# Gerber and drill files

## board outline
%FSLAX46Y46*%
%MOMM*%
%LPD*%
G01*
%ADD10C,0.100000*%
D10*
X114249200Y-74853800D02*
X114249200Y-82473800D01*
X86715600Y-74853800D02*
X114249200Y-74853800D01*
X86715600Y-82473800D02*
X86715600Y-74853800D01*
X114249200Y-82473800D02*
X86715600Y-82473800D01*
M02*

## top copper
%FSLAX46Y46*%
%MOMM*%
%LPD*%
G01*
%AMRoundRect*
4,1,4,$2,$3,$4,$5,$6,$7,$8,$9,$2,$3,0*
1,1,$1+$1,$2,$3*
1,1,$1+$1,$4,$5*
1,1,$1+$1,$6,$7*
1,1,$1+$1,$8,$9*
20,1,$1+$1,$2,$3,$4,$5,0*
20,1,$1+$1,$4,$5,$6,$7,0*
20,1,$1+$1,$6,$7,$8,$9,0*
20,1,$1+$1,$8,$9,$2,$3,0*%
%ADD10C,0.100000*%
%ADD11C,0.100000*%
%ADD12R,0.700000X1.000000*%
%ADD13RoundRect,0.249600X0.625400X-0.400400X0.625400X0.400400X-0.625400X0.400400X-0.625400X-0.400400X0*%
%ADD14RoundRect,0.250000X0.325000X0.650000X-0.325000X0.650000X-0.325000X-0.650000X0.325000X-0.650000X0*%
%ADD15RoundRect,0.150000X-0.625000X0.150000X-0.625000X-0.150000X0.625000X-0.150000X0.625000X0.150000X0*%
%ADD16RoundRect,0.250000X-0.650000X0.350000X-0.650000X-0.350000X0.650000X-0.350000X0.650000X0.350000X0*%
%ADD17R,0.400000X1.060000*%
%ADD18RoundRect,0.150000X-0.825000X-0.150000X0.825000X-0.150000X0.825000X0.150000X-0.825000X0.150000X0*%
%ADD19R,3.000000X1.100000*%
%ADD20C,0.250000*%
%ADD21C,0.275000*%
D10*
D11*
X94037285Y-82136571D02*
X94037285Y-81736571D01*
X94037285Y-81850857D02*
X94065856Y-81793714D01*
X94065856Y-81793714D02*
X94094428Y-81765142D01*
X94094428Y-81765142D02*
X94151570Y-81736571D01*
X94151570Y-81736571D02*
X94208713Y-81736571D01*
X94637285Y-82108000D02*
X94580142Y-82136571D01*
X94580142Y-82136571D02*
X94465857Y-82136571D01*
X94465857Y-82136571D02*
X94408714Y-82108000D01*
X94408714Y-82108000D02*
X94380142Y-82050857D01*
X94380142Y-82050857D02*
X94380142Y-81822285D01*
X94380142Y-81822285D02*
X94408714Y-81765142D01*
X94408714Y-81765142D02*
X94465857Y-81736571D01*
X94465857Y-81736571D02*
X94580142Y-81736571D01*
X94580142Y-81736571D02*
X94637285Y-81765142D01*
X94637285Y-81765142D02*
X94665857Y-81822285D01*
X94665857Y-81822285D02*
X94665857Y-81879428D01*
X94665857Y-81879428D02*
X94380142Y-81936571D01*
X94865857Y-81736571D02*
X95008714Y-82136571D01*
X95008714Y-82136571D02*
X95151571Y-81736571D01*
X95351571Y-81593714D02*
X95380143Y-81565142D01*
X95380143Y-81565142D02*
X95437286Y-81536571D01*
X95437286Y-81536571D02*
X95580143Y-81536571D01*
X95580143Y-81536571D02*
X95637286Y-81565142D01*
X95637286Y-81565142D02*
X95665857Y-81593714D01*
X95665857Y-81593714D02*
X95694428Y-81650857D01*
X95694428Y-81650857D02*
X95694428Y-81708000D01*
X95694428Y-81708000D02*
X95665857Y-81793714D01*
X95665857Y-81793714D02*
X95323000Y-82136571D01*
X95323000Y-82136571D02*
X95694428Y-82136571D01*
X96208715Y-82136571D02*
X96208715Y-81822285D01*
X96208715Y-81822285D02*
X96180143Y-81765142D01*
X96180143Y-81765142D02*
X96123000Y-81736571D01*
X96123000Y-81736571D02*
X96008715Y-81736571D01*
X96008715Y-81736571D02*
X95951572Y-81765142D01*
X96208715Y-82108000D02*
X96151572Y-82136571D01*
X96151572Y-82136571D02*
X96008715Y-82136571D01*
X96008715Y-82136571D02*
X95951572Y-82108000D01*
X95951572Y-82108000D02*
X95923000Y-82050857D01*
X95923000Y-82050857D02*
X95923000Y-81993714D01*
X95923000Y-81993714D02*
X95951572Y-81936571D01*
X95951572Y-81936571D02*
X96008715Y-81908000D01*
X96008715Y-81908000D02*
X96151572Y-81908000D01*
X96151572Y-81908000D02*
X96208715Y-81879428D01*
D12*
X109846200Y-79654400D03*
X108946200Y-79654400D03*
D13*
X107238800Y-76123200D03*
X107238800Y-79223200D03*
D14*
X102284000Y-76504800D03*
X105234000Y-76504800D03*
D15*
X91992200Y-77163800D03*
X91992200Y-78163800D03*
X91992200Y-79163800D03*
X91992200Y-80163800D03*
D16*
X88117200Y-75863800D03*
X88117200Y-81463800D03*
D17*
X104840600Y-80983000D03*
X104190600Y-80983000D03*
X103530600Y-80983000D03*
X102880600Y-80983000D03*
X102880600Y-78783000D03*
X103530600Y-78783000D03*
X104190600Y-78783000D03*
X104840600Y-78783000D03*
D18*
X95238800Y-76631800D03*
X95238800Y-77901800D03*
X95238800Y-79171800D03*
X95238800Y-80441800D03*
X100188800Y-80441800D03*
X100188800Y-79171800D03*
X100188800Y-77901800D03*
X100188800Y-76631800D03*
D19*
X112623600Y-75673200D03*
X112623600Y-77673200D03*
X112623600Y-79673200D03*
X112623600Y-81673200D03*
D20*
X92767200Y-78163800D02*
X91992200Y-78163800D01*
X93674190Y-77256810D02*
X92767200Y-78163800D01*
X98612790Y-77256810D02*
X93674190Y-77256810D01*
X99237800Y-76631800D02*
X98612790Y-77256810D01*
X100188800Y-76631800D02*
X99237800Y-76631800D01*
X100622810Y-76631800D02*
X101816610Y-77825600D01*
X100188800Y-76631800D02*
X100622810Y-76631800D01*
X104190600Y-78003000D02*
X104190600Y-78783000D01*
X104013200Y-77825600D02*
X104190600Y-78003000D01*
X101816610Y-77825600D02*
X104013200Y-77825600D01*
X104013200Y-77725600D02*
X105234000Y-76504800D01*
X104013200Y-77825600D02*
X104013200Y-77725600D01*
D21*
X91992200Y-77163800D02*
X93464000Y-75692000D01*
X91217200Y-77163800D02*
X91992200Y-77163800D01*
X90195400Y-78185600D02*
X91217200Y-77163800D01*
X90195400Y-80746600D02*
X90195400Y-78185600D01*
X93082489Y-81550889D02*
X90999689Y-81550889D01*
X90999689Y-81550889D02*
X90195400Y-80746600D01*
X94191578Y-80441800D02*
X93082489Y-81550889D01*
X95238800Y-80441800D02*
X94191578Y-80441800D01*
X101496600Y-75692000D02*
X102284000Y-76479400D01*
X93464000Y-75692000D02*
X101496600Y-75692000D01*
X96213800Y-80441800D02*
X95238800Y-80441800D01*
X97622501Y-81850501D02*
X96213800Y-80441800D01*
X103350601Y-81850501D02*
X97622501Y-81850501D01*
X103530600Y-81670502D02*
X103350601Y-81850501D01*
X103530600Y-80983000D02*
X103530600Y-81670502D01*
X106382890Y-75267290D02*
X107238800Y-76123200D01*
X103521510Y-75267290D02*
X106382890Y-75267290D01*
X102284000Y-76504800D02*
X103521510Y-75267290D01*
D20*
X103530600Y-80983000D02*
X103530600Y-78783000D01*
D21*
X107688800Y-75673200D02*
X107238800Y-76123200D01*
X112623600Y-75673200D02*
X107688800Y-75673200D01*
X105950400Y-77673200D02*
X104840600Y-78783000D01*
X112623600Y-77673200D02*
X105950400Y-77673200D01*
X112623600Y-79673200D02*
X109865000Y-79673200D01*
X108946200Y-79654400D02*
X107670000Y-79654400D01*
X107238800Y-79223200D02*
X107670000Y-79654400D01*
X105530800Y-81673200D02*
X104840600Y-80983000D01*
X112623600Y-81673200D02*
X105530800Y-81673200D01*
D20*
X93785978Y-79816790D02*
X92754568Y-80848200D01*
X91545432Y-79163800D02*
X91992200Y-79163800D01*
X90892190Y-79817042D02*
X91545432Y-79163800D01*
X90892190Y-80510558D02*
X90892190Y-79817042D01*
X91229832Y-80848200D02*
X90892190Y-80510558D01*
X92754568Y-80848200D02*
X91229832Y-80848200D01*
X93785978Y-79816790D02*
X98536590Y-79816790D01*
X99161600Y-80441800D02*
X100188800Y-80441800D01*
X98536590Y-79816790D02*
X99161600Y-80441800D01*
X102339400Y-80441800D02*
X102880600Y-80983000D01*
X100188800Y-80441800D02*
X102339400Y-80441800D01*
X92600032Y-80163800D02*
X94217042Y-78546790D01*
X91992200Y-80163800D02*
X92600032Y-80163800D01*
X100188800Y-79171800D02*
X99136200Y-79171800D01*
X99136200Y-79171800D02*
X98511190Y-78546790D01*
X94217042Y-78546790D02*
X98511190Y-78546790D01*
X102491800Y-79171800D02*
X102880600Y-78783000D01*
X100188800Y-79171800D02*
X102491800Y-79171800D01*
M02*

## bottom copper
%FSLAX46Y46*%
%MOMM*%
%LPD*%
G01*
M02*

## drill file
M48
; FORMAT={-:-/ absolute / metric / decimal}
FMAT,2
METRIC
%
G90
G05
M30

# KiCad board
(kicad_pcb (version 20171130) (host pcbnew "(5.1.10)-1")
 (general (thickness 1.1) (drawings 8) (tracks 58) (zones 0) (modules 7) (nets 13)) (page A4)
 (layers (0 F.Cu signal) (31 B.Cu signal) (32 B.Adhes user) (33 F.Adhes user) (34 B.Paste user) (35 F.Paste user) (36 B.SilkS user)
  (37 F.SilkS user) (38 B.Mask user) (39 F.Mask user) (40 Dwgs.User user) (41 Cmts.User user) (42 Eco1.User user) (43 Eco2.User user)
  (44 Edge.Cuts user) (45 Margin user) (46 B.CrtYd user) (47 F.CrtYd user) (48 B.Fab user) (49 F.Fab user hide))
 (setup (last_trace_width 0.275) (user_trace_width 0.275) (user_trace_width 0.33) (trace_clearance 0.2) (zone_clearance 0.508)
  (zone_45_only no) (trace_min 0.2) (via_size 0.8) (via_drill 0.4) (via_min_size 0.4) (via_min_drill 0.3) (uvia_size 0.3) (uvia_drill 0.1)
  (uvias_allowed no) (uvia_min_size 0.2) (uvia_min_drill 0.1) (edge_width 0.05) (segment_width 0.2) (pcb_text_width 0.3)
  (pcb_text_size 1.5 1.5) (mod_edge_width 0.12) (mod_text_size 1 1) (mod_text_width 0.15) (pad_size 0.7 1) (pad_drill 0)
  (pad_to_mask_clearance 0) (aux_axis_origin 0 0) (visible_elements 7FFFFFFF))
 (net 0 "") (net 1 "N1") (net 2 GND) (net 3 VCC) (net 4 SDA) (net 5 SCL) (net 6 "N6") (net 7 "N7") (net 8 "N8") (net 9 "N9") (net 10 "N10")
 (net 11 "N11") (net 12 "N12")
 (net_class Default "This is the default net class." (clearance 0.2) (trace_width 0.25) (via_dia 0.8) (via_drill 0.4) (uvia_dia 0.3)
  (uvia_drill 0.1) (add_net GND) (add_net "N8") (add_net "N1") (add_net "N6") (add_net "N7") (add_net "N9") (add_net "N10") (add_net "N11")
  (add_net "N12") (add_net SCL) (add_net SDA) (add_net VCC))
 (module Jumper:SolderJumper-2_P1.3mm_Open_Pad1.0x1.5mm (layer F.Cu) (at 109.2962 79.6544)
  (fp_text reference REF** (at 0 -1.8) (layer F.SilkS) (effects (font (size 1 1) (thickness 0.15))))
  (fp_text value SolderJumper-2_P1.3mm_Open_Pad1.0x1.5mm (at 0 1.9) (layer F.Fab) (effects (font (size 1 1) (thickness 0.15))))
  (pad 2 smd rect (at 0.55 0) (size 0.7 1) (layers F.Cu F.Mask) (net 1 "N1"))
  (pad 1 smd rect (at -0.35 0) (size 0.7 1) (layers F.Cu F.Mask) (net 1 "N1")))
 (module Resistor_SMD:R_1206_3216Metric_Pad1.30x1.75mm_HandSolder (layer F.Cu) (at 107.2388 77.6732 90)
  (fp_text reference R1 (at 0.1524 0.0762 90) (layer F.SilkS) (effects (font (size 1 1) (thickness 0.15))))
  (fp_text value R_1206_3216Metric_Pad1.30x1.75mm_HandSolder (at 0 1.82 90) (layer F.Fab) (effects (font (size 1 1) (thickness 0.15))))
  (pad 2 smd roundrect (at 1.55 0 90) (size 1.3 1.75) (layers F.Cu F.Paste F.Mask) (roundrect_rratio 0.192) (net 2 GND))
  (pad 1 smd roundrect (at -1.55 0 90) (size 1.3 1.75) (layers F.Cu F.Paste F.Mask) (roundrect_rratio 0.192) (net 1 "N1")))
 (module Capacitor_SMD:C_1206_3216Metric (layer F.Cu) (at 103.759 76.5048 180)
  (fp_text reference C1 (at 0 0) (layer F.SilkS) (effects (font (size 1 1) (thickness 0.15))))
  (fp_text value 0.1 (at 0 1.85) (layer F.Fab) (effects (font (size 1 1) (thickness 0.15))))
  (pad 2 smd roundrect (at 1.475 0 180) (size 1.15 1.8) (layers F.Cu F.Paste F.Mask) (roundrect_rratio 0.217391) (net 2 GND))
  (pad 1 smd roundrect (at -1.475 0 180) (size 1.15 1.8) (layers F.Cu F.Paste F.Mask) (roundrect_rratio 0.217391) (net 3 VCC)))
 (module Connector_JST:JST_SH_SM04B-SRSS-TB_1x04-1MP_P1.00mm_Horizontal (layer F.Cu) (at 89.9922 78.6638 270)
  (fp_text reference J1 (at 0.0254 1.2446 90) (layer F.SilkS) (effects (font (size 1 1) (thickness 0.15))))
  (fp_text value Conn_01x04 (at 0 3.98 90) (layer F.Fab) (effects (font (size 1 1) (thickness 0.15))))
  (pad 1 smd roundrect (at -1.5 -2 270) (size 0.6 1.55) (layers F.Cu F.Paste F.Mask) (roundrect_rratio 0.25) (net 2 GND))
  (pad 2 smd roundrect (at -0.5 -2 270) (size 0.6 1.55) (layers F.Cu F.Paste F.Mask) (roundrect_rratio 0.25) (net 3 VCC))
  (pad 3 smd roundrect (at 0.5 -2 270) (size 0.6 1.55) (layers F.Cu F.Paste F.Mask) (roundrect_rratio 0.25) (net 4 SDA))
  (pad 4 smd roundrect (at 1.5 -2 270) (size 0.6 1.55) (layers F.Cu F.Paste F.Mask) (roundrect_rratio 0.25) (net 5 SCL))
  (pad MP smd roundrect (at -2.8 1.875 270) (size 1.2 1.8) (layers F.Cu F.Paste F.Mask) (roundrect_rratio 0.208333))
  (pad MP smd roundrect (at 2.8 1.875 270) (size 1.2 1.8) (layers F.Cu F.Paste F.Mask) (roundrect_rratio 0.208333)))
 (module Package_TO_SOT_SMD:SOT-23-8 (layer F.Cu) (at 103.8606 79.883 270)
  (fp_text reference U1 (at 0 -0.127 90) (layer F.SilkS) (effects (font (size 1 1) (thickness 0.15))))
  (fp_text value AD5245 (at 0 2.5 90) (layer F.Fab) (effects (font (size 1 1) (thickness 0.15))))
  (pad 8 smd rect (at 1.1 -0.98 270) (size 1.06 0.4) (layers F.Cu F.Paste F.Mask) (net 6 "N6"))
  (pad 7 smd rect (at 1.1 -0.33 270) (size 1.06 0.4) (layers F.Cu F.Paste F.Mask) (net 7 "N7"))
  (pad 6 smd rect (at 1.1 0.33 270) (size 1.06 0.4) (layers F.Cu F.Paste F.Mask) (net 2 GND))
  (pad 5 smd rect (at 1.1 0.98 270) (size 1.06 0.4) (layers F.Cu F.Paste F.Mask) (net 4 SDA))
  (pad 4 smd rect (at -1.1 0.98 270) (size 1.06 0.4) (layers F.Cu F.Paste F.Mask) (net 5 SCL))
  (pad 3 smd rect (at -1.1 0.33 270) (size 1.06 0.4) (layers F.Cu F.Paste F.Mask) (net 2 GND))
  (pad 2 smd rect (at -1.1 -0.33 270) (size 1.06 0.4) (layers F.Cu F.Paste F.Mask) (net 3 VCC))
  (pad 1 smd rect (at -1.1 -0.98 270) (size 1.06 0.4) (layers F.Cu F.Paste F.Mask) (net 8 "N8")))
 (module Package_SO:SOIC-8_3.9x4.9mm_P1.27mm (layer F.Cu) (at 97.7138 78.5368)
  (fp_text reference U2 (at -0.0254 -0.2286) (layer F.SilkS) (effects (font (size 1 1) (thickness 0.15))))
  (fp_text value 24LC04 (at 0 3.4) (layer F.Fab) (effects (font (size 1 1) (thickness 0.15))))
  (pad 1 smd roundrect (at -2.475 -1.905) (size 1.95 0.6) (layers F.Cu F.Paste F.Mask) (roundrect_rratio 0.25) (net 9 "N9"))
  (pad 2 smd roundrect (at -2.475 -0.635) (size 1.95 0.6) (layers F.Cu F.Paste F.Mask) (roundrect_rratio 0.25) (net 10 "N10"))
  (pad 3 smd roundrect (at -2.475 0.635) (size 1.95 0.6) (layers F.Cu F.Paste F.Mask) (roundrect_rratio 0.25) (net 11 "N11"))
  (pad 4 smd roundrect (at -2.475 1.905) (size 1.95 0.6) (layers F.Cu F.Paste F.Mask) (roundrect_rratio 0.25) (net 2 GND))
  (pad 5 smd roundrect (at 2.475 1.905) (size 1.95 0.6) (layers F.Cu F.Paste F.Mask) (roundrect_rratio 0.25) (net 4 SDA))
  (pad 6 smd roundrect (at 2.475 0.635) (size 1.95 0.6) (layers F.Cu F.Paste F.Mask) (roundrect_rratio 0.25) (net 5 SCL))
  (pad 7 smd roundrect (at 2.475 -0.635) (size 1.95 0.6) (layers F.Cu F.Paste F.Mask) (roundrect_rratio 0.25) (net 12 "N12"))
  (pad 8 smd roundrect (at 2.475 -1.905) (size 1.95 0.6) (layers F.Cu F.Paste F.Mask) (roundrect_rratio 0.25) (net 3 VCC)))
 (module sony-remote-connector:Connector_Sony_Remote (layer F.Cu) (at 111.3536 77.6732 270)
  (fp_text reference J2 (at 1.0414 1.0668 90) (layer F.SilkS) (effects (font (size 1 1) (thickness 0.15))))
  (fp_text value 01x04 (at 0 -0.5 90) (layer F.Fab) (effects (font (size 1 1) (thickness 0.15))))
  (pad 1 smd rect (at -2 -1.27 270) (size 1.1 3) (layers F.Cu F.Mask) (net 2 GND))
  (pad 2 smd rect (at 0 -1.27 270) (size 1.1 3) (layers F.Cu F.Mask) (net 8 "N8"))
  (pad 3 smd rect (at 2 -1.27 270) (size 1.1 3) (layers F.Cu F.Mask) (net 1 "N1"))
  (pad 4 smd rect (at 4 -1.27 270) (size 1.1 3) (layers F.Cu F.Mask) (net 6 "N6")))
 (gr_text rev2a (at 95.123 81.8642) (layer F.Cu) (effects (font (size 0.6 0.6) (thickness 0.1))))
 (gr_line (start 114.2492 74.8538) (end 114.2492 82.4738) (layer Edge.Cuts) (width 0.1))
 (gr_line (start 86.7156 74.8538) (end 114.2492 74.8538) (layer Edge.Cuts) (width 0.1))
 (gr_line (start 86.7156 82.4738) (end 86.7156 74.8538) (layer Edge.Cuts) (width 0.1))
 (gr_line (start 114.2492 82.4738) (end 86.7156 82.4738) (layer Edge.Cuts) (width 0.1))
 (segment (start 92.7672 78.1638) (end 91.9922 78.1638) (width 0.25) (layer F.Cu) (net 3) (status 20))
 (segment (start 93.67419 77.25681) (end 92.7672 78.1638) (width 0.25) (layer F.Cu) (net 3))
 (segment (start 98.61279 77.25681) (end 93.67419 77.25681) (width 0.25) (layer F.Cu) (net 3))
 (segment (start 99.2378 76.6318) (end 98.61279 77.25681) (width 0.25) (layer F.Cu) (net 3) (status 10))
 (segment (start 100.1888 76.6318) (end 99.2378 76.6318) (width 0.25) (layer F.Cu) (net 3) (status 30))
 (segment (start 100.62281 76.6318) (end 101.81661 77.8256) (width 0.25) (layer F.Cu) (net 3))
 (segment (start 100.1888 76.6318) (end 100.62281 76.6318) (width 0.25) (layer F.Cu) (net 3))
 (segment (start 104.1906 78.003) (end 104.1906 78.783) (width 0.25) (layer F.Cu) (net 3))
 (segment (start 104.0132 77.8256) (end 104.1906 78.003) (width 0.25) (layer F.Cu) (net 3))
 (segment (start 101.81661 77.8256) (end 104.0132 77.8256) (width 0.25) (layer F.Cu) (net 3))
 (segment (start 104.0132 77.7256) (end 105.234 76.5048) (width 0.25) (layer F.Cu) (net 3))
 (segment (start 104.0132 77.8256) (end 104.0132 77.7256) (width 0.25) (layer F.Cu) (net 3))
 (segment (start 91.9922 77.1638) (end 93.464 75.692) (width 0.275) (layer F.Cu) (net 2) (status 10))
 (segment (start 91.2172 77.1638) (end 91.9922 77.1638) (width 0.275) (layer F.Cu) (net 2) (status 30))
 (segment (start 90.1954 78.1856) (end 91.2172 77.1638) (width 0.275) (layer F.Cu) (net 2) (status 20))
 (segment (start 90.1954 80.7466) (end 90.1954 78.1856) (width 0.275) (layer F.Cu) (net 2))
 (segment (start 93.082489 81.550889) (end 90.999689 81.550889) (width 0.275) (layer F.Cu) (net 2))
 (segment (start 90.999689 81.550889) (end 90.1954 80.7466) (width 0.275) (layer F.Cu) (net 2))
 (segment (start 94.191578 80.4418) (end 93.082489 81.550889) (width 0.275) (layer F.Cu) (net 2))
 (segment (start 95.2388 80.4418) (end 94.191578 80.4418) (width 0.275) (layer F.Cu) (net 2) (status 10))
 (segment (start 101.4966 75.692) (end 102.284 76.4794) (width 0.275) (layer F.Cu) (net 2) (status 20))
 (segment (start 93.464 75.692) (end 101.4966 75.692) (width 0.275) (layer F.Cu) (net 2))
 (segment (start 96.2138 80.4418) (end 95.2388 80.4418) (width 0.275) (layer F.Cu) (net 2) (status 20))
 (segment (start 97.622501 81.850501) (end 96.2138 80.4418) (width 0.275) (layer F.Cu) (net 2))
 (segment (start 103.350601 81.850501) (end 97.622501 81.850501) (width 0.275) (layer F.Cu) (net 2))
 (segment (start 103.5306 81.670502) (end 103.350601 81.850501) (width 0.275) (layer F.Cu) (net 2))
 (segment (start 103.5306 80.983) (end 103.5306 81.670502) (width 0.275) (layer F.Cu) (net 2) (status 10))
 (segment (start 106.38289 75.26729) (end 107.2388 76.1232) (width 0.275) (layer F.Cu) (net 2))
 (segment (start 103.52151 75.26729) (end 106.38289 75.26729) (width 0.275) (layer F.Cu) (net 2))
 (segment (start 102.284 76.5048) (end 103.52151 75.26729) (width 0.275) (layer F.Cu) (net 2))
 (segment (start 103.5306 80.983) (end 103.5306 78.783) (width 0.25) (layer F.Cu) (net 2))
 (segment (start 107.6888 75.6732) (end 107.2388 76.1232) (width 0.275) (layer F.Cu) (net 2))
 (segment (start 112.6236 75.6732) (end 107.6888 75.6732) (width 0.275) (layer F.Cu) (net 2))
 (segment (start 105.9504 77.6732) (end 104.8406 78.783) (width 0.275) (layer F.Cu) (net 8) (status 20))
 (segment (start 112.6236 77.6732) (end 105.9504 77.6732) (width 0.275) (layer F.Cu) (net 8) (status 10))
 (segment (start 112.6236 79.6732) (end 109.865 79.6732) (width 0.275) (layer F.Cu) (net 1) (status 30))
 (segment (start 108.9462 79.6544) (end 107.67 79.6544) (width 0.275) (layer F.Cu) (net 1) (status 30))
 (segment (start 107.2388 79.2232) (end 107.67 79.6544) (width 0.275) (layer F.Cu) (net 1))
 (segment (start 105.5308 81.6732) (end 104.8406 80.983) (width 0.275) (layer F.Cu) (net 6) (status 20))
 (segment (start 112.6236 81.6732) (end 105.5308 81.6732) (width 0.275) (layer F.Cu) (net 6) (status 10))
 (segment (start 93.785978 79.81679) (end 92.754568 80.8482) (width 0.25) (layer F.Cu) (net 4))
 (segment (start 91.545432 79.1638) (end 91.9922 79.1638) (width 0.25) (layer F.Cu) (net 4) (status 30))
 (segment (start 90.89219 79.817042) (end 91.545432 79.1638) (width 0.25) (layer F.Cu) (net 4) (status 20))
 (segment (start 90.89219 80.510558) (end 90.89219 79.817042) (width 0.25) (layer F.Cu) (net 4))
 (segment (start 91.229832 80.8482) (end 90.89219 80.510558) (width 0.25) (layer F.Cu) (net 4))
 (segment (start 92.754568 80.8482) (end 91.229832 80.8482) (width 0.25) (layer F.Cu) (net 4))
 (segment (start 93.785978 79.81679) (end 98.53659 79.81679) (width 0.25) (layer F.Cu) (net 4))
 (segment (start 99.1616 80.4418) (end 100.1888 80.4418) (width 0.25) (layer F.Cu) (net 4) (status 20))
 (segment (start 98.53659 79.81679) (end 99.1616 80.4418) (width 0.25) (layer F.Cu) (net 4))
 (segment (start 102.3394 80.4418) (end 102.8806 80.983) (width 0.25) (layer F.Cu) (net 4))
 (segment (start 100.1888 80.4418) (end 102.3394 80.4418) (width 0.25) (layer F.Cu) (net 4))
 (segment (start 92.600032 80.1638) (end 94.217042 78.54679) (width 0.25) (layer F.Cu) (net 5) (status 10))
 (segment (start 91.9922 80.1638) (end 92.600032 80.1638) (width 0.25) (layer F.Cu) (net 5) (status 30))
 (segment (start 100.1888 79.1718) (end 99.1362 79.1718) (width 0.25) (layer F.Cu) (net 5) (status 10))
 (segment (start 99.1362 79.1718) (end 98.51119 78.54679) (width 0.25) (layer F.Cu) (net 5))
 (segment (start 94.217042 78.54679) (end 98.51119 78.54679) (width 0.25) (layer F.Cu) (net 5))
 (segment (start 102.4918 79.1718) (end 102.8806 78.783) (width 0.25) (layer F.Cu) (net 5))
 (segment (start 100.1888 79.1718) (end 102.4918 79.1718) (width 0.25) (layer F.Cu) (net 5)))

